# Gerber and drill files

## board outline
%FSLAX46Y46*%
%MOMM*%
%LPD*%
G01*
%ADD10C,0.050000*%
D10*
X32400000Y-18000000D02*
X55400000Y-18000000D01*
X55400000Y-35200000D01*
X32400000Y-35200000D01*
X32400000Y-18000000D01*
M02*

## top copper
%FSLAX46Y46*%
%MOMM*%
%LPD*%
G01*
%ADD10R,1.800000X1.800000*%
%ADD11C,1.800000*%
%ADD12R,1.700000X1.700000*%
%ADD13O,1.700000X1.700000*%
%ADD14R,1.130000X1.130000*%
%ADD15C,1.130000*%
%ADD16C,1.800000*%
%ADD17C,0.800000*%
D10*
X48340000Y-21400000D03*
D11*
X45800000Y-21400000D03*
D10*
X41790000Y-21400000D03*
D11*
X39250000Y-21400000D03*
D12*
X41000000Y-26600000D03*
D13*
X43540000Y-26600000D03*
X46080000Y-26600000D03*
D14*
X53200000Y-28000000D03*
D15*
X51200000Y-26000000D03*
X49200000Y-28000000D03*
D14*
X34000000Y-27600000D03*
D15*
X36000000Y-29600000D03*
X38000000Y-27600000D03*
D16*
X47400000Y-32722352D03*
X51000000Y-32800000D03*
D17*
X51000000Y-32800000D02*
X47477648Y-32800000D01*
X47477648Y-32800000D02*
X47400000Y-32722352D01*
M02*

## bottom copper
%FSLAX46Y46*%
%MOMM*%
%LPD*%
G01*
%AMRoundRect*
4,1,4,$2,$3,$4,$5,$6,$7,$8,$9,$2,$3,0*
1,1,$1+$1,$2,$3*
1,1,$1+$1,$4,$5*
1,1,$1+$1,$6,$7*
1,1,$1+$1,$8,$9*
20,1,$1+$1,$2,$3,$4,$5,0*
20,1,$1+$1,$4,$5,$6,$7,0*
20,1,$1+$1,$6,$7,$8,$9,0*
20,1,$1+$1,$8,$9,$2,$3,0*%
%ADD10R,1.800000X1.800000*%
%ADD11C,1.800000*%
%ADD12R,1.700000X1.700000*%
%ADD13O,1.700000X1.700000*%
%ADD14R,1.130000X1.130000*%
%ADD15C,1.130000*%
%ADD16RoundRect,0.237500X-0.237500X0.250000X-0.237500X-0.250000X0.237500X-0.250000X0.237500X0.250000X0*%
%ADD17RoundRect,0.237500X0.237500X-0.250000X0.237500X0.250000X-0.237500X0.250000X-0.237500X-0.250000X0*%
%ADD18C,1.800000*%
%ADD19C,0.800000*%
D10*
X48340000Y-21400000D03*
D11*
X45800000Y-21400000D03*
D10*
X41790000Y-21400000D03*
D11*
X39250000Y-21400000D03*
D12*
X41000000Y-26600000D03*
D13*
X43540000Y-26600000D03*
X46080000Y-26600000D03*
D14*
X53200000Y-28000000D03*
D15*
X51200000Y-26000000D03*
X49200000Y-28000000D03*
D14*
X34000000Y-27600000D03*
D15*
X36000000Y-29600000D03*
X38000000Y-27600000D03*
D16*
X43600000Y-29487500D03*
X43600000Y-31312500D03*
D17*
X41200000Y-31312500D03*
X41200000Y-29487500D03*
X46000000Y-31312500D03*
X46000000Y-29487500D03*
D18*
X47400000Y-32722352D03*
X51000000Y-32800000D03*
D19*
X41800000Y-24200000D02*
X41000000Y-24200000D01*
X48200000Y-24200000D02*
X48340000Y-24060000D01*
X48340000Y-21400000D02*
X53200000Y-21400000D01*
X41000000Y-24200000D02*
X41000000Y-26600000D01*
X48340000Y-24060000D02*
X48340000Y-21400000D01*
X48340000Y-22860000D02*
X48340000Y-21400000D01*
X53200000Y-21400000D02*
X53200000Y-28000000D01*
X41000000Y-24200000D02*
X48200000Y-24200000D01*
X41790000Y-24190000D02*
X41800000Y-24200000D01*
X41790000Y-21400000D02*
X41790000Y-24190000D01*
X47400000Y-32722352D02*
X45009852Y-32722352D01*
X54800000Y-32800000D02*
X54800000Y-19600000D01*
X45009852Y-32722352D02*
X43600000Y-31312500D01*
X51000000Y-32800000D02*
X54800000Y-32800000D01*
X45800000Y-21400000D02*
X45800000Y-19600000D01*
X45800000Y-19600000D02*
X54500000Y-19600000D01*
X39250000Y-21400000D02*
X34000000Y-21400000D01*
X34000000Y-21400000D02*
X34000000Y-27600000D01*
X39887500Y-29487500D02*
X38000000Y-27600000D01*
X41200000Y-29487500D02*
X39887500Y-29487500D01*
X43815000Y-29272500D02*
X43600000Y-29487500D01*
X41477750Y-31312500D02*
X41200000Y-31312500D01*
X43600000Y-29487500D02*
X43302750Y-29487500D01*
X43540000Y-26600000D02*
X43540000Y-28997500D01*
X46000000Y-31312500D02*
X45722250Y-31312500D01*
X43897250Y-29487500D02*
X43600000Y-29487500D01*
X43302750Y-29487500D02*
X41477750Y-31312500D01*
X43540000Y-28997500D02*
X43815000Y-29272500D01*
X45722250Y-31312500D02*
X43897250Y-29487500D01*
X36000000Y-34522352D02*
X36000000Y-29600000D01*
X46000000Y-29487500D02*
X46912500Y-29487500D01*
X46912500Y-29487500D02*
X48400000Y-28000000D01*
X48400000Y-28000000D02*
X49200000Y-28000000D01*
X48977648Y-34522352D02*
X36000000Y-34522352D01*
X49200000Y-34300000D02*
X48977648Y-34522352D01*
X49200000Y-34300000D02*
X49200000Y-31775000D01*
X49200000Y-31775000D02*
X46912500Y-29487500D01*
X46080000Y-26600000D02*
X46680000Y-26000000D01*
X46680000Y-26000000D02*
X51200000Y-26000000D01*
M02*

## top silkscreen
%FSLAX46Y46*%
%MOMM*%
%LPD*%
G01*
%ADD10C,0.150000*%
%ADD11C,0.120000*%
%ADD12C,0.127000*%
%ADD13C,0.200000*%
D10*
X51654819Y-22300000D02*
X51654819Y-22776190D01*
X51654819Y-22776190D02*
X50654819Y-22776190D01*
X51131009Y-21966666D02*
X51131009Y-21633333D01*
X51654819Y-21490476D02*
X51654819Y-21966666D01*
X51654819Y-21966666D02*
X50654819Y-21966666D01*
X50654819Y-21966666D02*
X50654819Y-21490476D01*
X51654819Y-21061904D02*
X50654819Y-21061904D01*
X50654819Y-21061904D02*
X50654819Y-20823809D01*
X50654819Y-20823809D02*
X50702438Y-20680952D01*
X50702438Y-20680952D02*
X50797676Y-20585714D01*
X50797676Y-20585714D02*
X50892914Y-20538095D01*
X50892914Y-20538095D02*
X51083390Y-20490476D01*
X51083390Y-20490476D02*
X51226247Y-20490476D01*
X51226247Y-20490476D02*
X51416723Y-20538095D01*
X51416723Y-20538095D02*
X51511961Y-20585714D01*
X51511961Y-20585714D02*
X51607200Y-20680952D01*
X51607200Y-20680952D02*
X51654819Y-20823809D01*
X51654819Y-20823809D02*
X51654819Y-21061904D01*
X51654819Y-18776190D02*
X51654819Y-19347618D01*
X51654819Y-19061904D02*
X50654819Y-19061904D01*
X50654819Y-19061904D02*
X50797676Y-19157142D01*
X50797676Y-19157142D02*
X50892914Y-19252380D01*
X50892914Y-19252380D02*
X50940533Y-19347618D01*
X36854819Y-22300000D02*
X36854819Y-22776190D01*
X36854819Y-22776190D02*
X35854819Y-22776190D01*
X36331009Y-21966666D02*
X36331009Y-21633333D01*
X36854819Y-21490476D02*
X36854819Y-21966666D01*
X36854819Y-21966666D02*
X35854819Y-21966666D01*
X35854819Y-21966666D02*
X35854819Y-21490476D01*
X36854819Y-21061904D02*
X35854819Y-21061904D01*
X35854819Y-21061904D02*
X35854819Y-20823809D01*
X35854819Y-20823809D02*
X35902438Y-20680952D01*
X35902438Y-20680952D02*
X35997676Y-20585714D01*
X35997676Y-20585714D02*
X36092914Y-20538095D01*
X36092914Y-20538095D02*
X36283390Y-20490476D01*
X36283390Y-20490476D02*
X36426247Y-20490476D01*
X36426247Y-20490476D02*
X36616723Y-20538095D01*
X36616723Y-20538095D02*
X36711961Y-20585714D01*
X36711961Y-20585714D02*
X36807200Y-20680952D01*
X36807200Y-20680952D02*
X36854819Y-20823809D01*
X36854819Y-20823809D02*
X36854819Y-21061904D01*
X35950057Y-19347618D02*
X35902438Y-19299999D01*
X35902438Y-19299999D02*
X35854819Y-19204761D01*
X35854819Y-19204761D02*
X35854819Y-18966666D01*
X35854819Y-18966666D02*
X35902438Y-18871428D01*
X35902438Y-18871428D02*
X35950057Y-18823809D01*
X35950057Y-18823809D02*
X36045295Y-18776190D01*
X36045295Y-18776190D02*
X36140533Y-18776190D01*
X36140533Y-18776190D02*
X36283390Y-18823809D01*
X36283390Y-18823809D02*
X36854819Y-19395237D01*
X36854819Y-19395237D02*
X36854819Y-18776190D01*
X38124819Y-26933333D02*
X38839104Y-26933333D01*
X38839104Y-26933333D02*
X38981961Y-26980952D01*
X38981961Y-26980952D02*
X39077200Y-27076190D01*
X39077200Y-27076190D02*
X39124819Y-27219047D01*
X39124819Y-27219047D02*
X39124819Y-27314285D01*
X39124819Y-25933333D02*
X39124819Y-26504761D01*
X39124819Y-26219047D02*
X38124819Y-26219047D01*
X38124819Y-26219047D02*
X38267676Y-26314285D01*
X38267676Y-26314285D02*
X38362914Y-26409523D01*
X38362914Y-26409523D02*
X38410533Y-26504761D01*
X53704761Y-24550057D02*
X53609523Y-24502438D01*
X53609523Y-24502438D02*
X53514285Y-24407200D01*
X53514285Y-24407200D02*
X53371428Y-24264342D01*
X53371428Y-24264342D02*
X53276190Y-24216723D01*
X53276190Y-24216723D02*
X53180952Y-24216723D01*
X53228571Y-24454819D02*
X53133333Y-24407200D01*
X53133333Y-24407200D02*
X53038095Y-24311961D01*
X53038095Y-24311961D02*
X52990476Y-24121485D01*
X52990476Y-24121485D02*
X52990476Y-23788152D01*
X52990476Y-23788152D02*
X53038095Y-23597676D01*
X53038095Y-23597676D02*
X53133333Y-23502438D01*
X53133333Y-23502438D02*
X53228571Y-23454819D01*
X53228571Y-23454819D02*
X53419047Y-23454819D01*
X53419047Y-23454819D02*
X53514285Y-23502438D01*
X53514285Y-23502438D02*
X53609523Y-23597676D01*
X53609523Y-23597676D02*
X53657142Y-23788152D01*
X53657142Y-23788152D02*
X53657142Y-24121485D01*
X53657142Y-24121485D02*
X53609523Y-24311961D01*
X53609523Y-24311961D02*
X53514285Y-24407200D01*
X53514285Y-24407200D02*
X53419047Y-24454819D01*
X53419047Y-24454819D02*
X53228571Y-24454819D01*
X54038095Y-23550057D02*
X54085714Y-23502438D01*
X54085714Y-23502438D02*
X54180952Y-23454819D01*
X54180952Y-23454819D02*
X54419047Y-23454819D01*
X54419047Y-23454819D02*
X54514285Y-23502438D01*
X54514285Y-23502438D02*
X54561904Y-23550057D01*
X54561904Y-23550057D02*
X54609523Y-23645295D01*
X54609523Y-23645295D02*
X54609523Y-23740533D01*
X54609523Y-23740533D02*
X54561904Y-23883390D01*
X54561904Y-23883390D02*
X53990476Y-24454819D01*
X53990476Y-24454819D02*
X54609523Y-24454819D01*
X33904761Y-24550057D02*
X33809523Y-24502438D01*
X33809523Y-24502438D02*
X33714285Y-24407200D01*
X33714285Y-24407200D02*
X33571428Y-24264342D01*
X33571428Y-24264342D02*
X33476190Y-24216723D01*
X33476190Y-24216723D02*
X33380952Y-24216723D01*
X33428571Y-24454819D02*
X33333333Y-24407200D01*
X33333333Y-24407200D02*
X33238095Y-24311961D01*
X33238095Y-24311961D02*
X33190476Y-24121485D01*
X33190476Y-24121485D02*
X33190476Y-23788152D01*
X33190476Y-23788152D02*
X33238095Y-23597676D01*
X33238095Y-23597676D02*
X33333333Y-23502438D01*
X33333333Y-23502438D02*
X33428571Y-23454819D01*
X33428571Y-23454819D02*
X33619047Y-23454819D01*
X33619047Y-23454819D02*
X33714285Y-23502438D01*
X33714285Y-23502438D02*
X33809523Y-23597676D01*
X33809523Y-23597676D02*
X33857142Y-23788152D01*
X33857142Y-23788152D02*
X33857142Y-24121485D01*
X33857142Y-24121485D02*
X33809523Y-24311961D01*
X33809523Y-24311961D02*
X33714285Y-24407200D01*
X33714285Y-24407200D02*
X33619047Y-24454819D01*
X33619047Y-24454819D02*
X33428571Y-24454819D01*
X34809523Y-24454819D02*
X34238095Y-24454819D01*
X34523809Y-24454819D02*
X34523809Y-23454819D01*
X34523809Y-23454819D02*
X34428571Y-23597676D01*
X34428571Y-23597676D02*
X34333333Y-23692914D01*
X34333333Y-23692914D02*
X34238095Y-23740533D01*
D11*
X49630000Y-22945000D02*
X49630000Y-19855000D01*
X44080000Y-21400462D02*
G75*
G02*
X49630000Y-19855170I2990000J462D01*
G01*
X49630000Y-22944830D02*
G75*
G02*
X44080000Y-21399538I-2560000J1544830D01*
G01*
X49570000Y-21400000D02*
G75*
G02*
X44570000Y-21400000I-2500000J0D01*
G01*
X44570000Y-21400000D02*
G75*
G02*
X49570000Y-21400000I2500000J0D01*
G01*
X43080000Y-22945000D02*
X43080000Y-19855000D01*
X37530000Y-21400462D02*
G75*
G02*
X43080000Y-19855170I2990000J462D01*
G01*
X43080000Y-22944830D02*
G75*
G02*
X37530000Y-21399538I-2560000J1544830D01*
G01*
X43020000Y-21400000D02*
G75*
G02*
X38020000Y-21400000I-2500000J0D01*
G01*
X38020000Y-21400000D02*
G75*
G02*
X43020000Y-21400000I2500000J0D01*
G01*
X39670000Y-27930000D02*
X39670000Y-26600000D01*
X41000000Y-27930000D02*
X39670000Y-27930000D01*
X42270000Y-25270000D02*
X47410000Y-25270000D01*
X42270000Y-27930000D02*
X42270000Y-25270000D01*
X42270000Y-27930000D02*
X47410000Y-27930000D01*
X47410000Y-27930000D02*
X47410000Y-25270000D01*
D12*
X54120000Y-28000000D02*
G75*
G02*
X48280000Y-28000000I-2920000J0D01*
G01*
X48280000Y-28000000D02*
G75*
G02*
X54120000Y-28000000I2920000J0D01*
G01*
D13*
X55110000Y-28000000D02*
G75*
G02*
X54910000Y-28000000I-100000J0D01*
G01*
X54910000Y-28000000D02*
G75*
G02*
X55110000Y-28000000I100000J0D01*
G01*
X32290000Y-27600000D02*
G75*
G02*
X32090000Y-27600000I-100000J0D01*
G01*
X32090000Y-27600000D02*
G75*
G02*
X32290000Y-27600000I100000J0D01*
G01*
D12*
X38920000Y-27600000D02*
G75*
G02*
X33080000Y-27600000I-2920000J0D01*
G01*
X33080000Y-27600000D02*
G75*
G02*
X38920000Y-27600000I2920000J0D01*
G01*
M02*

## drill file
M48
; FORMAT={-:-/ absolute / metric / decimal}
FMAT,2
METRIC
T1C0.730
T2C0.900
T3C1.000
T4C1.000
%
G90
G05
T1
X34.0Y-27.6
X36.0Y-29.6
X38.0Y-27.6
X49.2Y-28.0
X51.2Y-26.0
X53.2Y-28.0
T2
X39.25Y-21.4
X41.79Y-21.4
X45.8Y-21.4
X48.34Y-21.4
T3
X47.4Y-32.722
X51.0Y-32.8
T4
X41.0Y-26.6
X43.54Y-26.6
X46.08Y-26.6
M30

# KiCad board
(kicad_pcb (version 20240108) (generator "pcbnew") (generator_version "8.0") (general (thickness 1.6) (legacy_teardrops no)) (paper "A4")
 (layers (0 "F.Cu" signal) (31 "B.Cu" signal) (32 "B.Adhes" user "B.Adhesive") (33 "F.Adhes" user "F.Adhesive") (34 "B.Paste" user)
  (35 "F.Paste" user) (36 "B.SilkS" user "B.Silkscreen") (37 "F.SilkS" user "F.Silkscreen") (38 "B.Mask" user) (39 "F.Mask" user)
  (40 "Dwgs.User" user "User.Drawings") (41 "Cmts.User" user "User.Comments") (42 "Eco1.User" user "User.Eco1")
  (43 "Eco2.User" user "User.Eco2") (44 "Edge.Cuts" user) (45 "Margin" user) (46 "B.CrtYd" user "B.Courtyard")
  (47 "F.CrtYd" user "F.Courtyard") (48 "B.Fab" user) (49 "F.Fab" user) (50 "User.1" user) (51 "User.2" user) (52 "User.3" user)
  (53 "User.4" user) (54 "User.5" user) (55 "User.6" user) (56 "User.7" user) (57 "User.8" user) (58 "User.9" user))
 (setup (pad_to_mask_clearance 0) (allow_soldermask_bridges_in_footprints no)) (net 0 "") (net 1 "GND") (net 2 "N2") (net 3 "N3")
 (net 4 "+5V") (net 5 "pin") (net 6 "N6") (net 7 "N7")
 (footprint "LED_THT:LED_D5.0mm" (layer "F.Cu") (at 48.34 21.4 180)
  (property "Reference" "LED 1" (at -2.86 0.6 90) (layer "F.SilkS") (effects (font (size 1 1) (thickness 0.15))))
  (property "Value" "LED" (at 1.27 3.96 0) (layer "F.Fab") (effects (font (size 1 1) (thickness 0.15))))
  (fp_line (start -1.29 -1.545) (end -1.29 1.545) (stroke (width 0.12) (type solid)) (layer "F.SilkS"))
  (fp_arc (start 4.26 -0.000462) (mid 2.072002 2.880433) (end -1.29 1.54483) (stroke (width 0.12) (type solid)) (layer "F.SilkS"))
  (fp_arc (start -1.29 -1.54483) (mid 2.072002 -2.880433) (end 4.26 0.000462) (stroke (width 0.12) (type solid)) (layer "F.SilkS"))
  (fp_circle (center 1.27 0) (end 3.77 0) (stroke (width 0.12) (type solid)) (fill none) (layer "F.SilkS"))
  (pad "1" thru_hole rect (at 0 0 180) (size 1.8 1.8) (drill 0.9) (layers "*.Cu" "*.Mask") (remove_unused_layers no) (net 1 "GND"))
  (pad "2" thru_hole circle (at 2.54 0 180) (size 1.8 1.8) (drill 0.9) (layers "*.Cu" "*.Mask") (remove_unused_layers no) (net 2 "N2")))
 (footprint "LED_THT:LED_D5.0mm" (layer "F.Cu") (at 41.79 21.4 180)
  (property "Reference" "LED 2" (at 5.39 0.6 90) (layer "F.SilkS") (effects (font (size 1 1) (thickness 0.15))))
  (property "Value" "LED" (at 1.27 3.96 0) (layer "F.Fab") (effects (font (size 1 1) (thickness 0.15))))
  (fp_line (start -1.29 -1.545) (end -1.29 1.545) (stroke (width 0.12) (type solid)) (layer "F.SilkS"))
  (fp_arc (start 4.26 -0.000462) (mid 2.072002 2.880433) (end -1.29 1.54483) (stroke (width 0.12) (type solid)) (layer "F.SilkS"))
  (fp_arc (start -1.29 -1.54483) (mid 2.072002 -2.880433) (end 4.26 0.000462) (stroke (width 0.12) (type solid)) (layer "F.SilkS"))
  (fp_circle (center 1.27 0) (end 3.77 0) (stroke (width 0.12) (type solid)) (fill none) (layer "F.SilkS"))
  (pad "1" thru_hole rect (at 0 0 180) (size 1.8 1.8) (drill 0.9) (layers "*.Cu" "*.Mask") (remove_unused_layers no) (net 1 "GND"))
  (pad "2" thru_hole circle (at 2.54 0 180) (size 1.8 1.8) (drill 0.9) (layers "*.Cu" "*.Mask") (remove_unused_layers no) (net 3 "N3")))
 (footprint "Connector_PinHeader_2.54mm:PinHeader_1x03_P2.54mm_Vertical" (layer "F.Cu") (at 41 26.6 90)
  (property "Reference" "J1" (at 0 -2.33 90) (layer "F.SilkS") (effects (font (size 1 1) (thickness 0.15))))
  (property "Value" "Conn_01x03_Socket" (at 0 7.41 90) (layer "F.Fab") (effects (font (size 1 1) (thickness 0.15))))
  (fp_line (start -1.33 -1.33) (end 0 -1.33) (stroke (width 0.12) (type solid)) (layer "F.SilkS"))
  (fp_line (start -1.33 0) (end -1.33 -1.33) (stroke (width 0.12) (type solid)) (layer "F.SilkS"))
  (fp_line (start 1.33 1.27) (end 1.33 6.41) (stroke (width 0.12) (type solid)) (layer "F.SilkS"))
  (fp_line (start -1.33 1.27) (end 1.33 1.27) (stroke (width 0.12) (type solid)) (layer "F.SilkS"))
  (fp_line (start -1.33 1.27) (end -1.33 6.41) (stroke (width 0.12) (type solid)) (layer "F.SilkS"))
  (fp_line (start -1.33 6.41) (end 1.33 6.41) (stroke (width 0.12) (type solid)) (layer "F.SilkS"))
  (pad "1" thru_hole rect (at 0 0 90) (size 1.7 1.7) (drill 1) (layers "*.Cu" "*.Mask") (remove_unused_layers no) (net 1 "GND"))
  (pad "2" thru_hole oval (at 0 2.54 90) (size 1.7 1.7) (drill 1) (layers "*.Cu" "*.Mask") (remove_unused_layers no) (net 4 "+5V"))
  (pad "3" thru_hole oval (at 0 5.08 90) (size 1.7 1.7) (drill 1) (layers "*.Cu" "*.Mask") (remove_unused_layers no) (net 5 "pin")))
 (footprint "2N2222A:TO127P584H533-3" (layer "F.Cu") (at 51.2 28 180)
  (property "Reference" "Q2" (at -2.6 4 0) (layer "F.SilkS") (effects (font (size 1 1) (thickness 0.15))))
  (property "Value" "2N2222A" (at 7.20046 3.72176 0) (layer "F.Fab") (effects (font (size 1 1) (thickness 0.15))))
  (fp_circle (center 0 0) (end 2.92 0) (stroke (width 0.127) (type solid)) (fill none) (layer "F.SilkS"))
  (fp_circle (center -3.81 0) (end -3.71 0) (stroke (width 0.2) (type solid)) (fill none) (layer "F.SilkS"))
  (pad "1" thru_hole rect (at -2 0 180) (size 1.13 1.13) (drill 0.73) (layers "*.Cu" "*.Mask") (remove_unused_layers no) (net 1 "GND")
   (solder_mask_margin 0.102))
  (pad "2" thru_hole circle (at 0 2 180) (size 1.13 1.13) (drill 0.73) (layers "*.Cu" "*.Mask") (remove_unused_layers no) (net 5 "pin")
   (solder_mask_margin 0.102))
  (pad "3" thru_hole circle (at 2 0 180) (size 1.13 1.13) (drill 0.73) (layers "*.Cu" "*.Mask") (remove_unused_layers no) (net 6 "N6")
   (solder_mask_margin 0.102)))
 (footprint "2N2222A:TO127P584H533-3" (layer "F.Cu") (at 36 27.6)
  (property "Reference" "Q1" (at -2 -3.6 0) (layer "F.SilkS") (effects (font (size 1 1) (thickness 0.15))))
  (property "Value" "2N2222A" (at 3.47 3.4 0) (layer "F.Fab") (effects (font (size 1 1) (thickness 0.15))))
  (fp_circle (center -3.81 0) (end -3.71 0) (stroke (width 0.2) (type solid)) (fill none) (layer "F.SilkS"))
  (fp_circle (center 0 0) (end 2.92 0) (stroke (width 0.127) (type solid)) (fill none) (layer "F.SilkS"))
  (pad "1" thru_hole rect (at -2 0) (size 1.13 1.13) (drill 0.73) (layers "*.Cu" "*.Mask") (remove_unused_layers no) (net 3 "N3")
   (solder_mask_margin 0.102))
  (pad "2" thru_hole circle (at 0 2) (size 1.13 1.13) (drill 0.73) (layers "*.Cu" "*.Mask") (remove_unused_layers no) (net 6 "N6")
   (solder_mask_margin 0.102))
  (pad "3" thru_hole circle (at 2 0) (size 1.13 1.13) (drill 0.73) (layers "*.Cu" "*.Mask") (remove_unused_layers no) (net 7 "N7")
   (solder_mask_margin 0.102)))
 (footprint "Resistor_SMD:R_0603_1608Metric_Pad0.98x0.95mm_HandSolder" (layer "B.Cu") (at 43.6 30.4 -90)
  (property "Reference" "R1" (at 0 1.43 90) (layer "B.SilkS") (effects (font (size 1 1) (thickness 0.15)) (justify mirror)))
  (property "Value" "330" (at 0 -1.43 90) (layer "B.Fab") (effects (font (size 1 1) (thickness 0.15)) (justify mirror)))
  (pad "1" smd roundrect (at -0.9125 0 270) (size 0.975 0.95) (layers "B.Cu" "B.Paste" "B.Mask") (roundrect_rratio 0.25) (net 4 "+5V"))
  (pad "2" smd roundrect (at 0.9125 0 270) (size 0.975 0.95) (layers "B.Cu" "B.Paste" "B.Mask") (roundrect_rratio 0.25) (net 2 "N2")))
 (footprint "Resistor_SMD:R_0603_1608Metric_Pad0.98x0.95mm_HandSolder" (layer "B.Cu") (at 41.2 30.4 90)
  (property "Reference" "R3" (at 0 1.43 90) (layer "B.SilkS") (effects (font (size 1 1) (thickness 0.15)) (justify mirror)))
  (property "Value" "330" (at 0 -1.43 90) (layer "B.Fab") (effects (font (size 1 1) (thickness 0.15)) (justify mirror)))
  (pad "1" smd roundrect (at -0.9125 0 90) (size 0.975 0.95) (layers "B.Cu" "B.Paste" "B.Mask") (roundrect_rratio 0.25) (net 4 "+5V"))
  (pad "2" smd roundrect (at 0.9125 0 90) (size 0.975 0.95) (layers "B.Cu" "B.Paste" "B.Mask") (roundrect_rratio 0.25) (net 7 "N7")))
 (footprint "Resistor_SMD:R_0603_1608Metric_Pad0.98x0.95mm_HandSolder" (layer "B.Cu") (at 46 30.4 90)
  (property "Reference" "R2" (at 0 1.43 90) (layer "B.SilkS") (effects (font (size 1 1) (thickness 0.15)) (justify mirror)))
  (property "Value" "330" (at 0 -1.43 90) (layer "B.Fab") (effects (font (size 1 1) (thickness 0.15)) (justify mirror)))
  (pad "1" smd roundrect (at -0.9125 0 90) (size 0.975 0.95) (layers "B.Cu" "B.Paste" "B.Mask") (roundrect_rratio 0.25) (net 4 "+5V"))
  (pad "2" smd roundrect (at 0.9125 0 90) (size 0.975 0.95) (layers "B.Cu" "B.Paste" "B.Mask") (roundrect_rratio 0.25) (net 6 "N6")))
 (gr_rect (start 32.4 18) (end 55.4 35.2) (stroke (width 0.05) (type default)) (fill none) (layer "Edge.Cuts"))
 (segment (start 41.8 24.2) (end 41 24.2) (width 0.8) (layer "B.Cu") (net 1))
 (segment (start 48.2 24.2) (end 48.34 24.06) (width 0.8) (layer "B.Cu") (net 1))
 (segment (start 48.34 21.4) (end 53.2 21.4) (width 0.8) (layer "B.Cu") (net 1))
 (segment (start 41 24.2) (end 41 26.6) (width 0.8) (layer "B.Cu") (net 1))
 (segment (start 48.34 24.06) (end 48.34 21.4) (width 0.8) (layer "B.Cu") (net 1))
 (segment (start 48.34 22.86) (end 48.34 21.4) (width 0.8) (layer "B.Cu") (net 1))
 (segment (start 53.2 21.4) (end 53.2 28) (width 0.8) (layer "B.Cu") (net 1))
 (segment (start 41 24.2) (end 48.2 24.2) (width 0.8) (layer "B.Cu") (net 1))
 (segment (start 41.79 24.19) (end 41.8 24.2) (width 0.8) (layer "B.Cu") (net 1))
 (segment (start 41.79 21.4) (end 41.79 24.19) (width 0.8) (layer "B.Cu") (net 1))
 (segment (start 51 32.8) (end 47.477648 32.8) (width 0.8) (layer "F.Cu") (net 2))
 (segment (start 47.477648 32.8) (end 47.4 32.722352) (width 0.8) (layer "F.Cu") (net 2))
 (via (at 47.4 32.722352) (size 1.8) (drill 1) (layers "F.Cu" "B.Cu") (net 2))
 (via (at 51 32.8) (size 1.8) (drill 1) (layers "F.Cu" "B.Cu") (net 2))
 (segment (start 47.4 32.722352) (end 45.009852 32.722352) (width 0.8) (layer "B.Cu") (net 2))
 (segment (start 54.8 32.8) (end 54.8 19.6) (width 0.8) (layer "B.Cu") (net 2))
 (segment (start 45.009852 32.722352) (end 43.6 31.3125) (width 0.8) (layer "B.Cu") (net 2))
 (segment (start 51 32.8) (end 54.8 32.8) (width 0.8) (layer "B.Cu") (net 2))
 (segment (start 45.8 21.4) (end 45.8 19.6) (width 0.8) (layer "B.Cu") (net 2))
 (segment (start 45.8 19.6) (end 54.5 19.6) (width 0.8) (layer "B.Cu") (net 2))
 (segment (start 39.25 21.4) (end 34 21.4) (width 0.8) (layer "B.Cu") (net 3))
 (segment (start 34 21.4) (end 34 27.6) (width 0.8) (layer "B.Cu") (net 3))
 (segment (start 39.8875 29.4875) (end 38 27.6) (width 0.8) (layer "B.Cu") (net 7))
 (segment (start 41.2 29.4875) (end 39.8875 29.4875) (width 0.8) (layer "B.Cu") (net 7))
 (segment (start 43.815 29.2725) (end 43.6 29.4875) (width 0.8) (layer "B.Cu") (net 4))
 (segment (start 41.47775 31.3125) (end 41.2 31.3125) (width 0.8) (layer "B.Cu") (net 4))
 (segment (start 43.6 29.4875) (end 43.30275 29.4875) (width 0.8) (layer "B.Cu") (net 4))
 (segment (start 43.54 26.6) (end 43.54 28.9975) (width 0.8) (layer "B.Cu") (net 4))
 (segment (start 46 31.3125) (end 45.72225 31.3125) (width 0.8) (layer "B.Cu") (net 4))
 (segment (start 43.89725 29.4875) (end 43.6 29.4875) (width 0.8) (layer "B.Cu") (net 4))
 (segment (start 43.30275 29.4875) (end 41.47775 31.3125) (width 0.8) (layer "B.Cu") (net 4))
 (segment (start 43.54 28.9975) (end 43.815 29.2725) (width 0.8) (layer "B.Cu") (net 4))
 (segment (start 45.72225 31.3125) (end 43.89725 29.4875) (width 0.8) (layer "B.Cu") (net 4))
 (segment (start 36 34.522352) (end 36 29.6) (width 0.8) (layer "B.Cu") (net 6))
 (segment (start 46 29.4875) (end 46.9125 29.4875) (width 0.8) (layer "B.Cu") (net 6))
 (segment (start 46.9125 29.4875) (end 48.4 28) (width 0.8) (layer "B.Cu") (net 6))
 (segment (start 48.4 28) (end 49.2 28) (width 0.8) (layer "B.Cu") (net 6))
 (segment (start 48.977648 34.522352) (end 36 34.522352) (width 0.8) (layer "B.Cu") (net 6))
 (segment (start 49.2 34.3) (end 48.977648 34.522352) (width 0.8) (layer "B.Cu") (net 6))
 (segment (start 49.2 34.3) (end 49.2 31.775) (width 0.8) (layer "B.Cu") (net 6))
 (segment (start 49.2 31.775) (end 46.9125 29.4875) (width 0.8) (layer "B.Cu") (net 6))
 (segment (start 46.08 26.6) (end 46.68 26) (width 0.8) (layer "B.Cu") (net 5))
 (segment (start 46.68 26) (end 51.2 26) (width 0.8) (layer "B.Cu") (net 5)))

